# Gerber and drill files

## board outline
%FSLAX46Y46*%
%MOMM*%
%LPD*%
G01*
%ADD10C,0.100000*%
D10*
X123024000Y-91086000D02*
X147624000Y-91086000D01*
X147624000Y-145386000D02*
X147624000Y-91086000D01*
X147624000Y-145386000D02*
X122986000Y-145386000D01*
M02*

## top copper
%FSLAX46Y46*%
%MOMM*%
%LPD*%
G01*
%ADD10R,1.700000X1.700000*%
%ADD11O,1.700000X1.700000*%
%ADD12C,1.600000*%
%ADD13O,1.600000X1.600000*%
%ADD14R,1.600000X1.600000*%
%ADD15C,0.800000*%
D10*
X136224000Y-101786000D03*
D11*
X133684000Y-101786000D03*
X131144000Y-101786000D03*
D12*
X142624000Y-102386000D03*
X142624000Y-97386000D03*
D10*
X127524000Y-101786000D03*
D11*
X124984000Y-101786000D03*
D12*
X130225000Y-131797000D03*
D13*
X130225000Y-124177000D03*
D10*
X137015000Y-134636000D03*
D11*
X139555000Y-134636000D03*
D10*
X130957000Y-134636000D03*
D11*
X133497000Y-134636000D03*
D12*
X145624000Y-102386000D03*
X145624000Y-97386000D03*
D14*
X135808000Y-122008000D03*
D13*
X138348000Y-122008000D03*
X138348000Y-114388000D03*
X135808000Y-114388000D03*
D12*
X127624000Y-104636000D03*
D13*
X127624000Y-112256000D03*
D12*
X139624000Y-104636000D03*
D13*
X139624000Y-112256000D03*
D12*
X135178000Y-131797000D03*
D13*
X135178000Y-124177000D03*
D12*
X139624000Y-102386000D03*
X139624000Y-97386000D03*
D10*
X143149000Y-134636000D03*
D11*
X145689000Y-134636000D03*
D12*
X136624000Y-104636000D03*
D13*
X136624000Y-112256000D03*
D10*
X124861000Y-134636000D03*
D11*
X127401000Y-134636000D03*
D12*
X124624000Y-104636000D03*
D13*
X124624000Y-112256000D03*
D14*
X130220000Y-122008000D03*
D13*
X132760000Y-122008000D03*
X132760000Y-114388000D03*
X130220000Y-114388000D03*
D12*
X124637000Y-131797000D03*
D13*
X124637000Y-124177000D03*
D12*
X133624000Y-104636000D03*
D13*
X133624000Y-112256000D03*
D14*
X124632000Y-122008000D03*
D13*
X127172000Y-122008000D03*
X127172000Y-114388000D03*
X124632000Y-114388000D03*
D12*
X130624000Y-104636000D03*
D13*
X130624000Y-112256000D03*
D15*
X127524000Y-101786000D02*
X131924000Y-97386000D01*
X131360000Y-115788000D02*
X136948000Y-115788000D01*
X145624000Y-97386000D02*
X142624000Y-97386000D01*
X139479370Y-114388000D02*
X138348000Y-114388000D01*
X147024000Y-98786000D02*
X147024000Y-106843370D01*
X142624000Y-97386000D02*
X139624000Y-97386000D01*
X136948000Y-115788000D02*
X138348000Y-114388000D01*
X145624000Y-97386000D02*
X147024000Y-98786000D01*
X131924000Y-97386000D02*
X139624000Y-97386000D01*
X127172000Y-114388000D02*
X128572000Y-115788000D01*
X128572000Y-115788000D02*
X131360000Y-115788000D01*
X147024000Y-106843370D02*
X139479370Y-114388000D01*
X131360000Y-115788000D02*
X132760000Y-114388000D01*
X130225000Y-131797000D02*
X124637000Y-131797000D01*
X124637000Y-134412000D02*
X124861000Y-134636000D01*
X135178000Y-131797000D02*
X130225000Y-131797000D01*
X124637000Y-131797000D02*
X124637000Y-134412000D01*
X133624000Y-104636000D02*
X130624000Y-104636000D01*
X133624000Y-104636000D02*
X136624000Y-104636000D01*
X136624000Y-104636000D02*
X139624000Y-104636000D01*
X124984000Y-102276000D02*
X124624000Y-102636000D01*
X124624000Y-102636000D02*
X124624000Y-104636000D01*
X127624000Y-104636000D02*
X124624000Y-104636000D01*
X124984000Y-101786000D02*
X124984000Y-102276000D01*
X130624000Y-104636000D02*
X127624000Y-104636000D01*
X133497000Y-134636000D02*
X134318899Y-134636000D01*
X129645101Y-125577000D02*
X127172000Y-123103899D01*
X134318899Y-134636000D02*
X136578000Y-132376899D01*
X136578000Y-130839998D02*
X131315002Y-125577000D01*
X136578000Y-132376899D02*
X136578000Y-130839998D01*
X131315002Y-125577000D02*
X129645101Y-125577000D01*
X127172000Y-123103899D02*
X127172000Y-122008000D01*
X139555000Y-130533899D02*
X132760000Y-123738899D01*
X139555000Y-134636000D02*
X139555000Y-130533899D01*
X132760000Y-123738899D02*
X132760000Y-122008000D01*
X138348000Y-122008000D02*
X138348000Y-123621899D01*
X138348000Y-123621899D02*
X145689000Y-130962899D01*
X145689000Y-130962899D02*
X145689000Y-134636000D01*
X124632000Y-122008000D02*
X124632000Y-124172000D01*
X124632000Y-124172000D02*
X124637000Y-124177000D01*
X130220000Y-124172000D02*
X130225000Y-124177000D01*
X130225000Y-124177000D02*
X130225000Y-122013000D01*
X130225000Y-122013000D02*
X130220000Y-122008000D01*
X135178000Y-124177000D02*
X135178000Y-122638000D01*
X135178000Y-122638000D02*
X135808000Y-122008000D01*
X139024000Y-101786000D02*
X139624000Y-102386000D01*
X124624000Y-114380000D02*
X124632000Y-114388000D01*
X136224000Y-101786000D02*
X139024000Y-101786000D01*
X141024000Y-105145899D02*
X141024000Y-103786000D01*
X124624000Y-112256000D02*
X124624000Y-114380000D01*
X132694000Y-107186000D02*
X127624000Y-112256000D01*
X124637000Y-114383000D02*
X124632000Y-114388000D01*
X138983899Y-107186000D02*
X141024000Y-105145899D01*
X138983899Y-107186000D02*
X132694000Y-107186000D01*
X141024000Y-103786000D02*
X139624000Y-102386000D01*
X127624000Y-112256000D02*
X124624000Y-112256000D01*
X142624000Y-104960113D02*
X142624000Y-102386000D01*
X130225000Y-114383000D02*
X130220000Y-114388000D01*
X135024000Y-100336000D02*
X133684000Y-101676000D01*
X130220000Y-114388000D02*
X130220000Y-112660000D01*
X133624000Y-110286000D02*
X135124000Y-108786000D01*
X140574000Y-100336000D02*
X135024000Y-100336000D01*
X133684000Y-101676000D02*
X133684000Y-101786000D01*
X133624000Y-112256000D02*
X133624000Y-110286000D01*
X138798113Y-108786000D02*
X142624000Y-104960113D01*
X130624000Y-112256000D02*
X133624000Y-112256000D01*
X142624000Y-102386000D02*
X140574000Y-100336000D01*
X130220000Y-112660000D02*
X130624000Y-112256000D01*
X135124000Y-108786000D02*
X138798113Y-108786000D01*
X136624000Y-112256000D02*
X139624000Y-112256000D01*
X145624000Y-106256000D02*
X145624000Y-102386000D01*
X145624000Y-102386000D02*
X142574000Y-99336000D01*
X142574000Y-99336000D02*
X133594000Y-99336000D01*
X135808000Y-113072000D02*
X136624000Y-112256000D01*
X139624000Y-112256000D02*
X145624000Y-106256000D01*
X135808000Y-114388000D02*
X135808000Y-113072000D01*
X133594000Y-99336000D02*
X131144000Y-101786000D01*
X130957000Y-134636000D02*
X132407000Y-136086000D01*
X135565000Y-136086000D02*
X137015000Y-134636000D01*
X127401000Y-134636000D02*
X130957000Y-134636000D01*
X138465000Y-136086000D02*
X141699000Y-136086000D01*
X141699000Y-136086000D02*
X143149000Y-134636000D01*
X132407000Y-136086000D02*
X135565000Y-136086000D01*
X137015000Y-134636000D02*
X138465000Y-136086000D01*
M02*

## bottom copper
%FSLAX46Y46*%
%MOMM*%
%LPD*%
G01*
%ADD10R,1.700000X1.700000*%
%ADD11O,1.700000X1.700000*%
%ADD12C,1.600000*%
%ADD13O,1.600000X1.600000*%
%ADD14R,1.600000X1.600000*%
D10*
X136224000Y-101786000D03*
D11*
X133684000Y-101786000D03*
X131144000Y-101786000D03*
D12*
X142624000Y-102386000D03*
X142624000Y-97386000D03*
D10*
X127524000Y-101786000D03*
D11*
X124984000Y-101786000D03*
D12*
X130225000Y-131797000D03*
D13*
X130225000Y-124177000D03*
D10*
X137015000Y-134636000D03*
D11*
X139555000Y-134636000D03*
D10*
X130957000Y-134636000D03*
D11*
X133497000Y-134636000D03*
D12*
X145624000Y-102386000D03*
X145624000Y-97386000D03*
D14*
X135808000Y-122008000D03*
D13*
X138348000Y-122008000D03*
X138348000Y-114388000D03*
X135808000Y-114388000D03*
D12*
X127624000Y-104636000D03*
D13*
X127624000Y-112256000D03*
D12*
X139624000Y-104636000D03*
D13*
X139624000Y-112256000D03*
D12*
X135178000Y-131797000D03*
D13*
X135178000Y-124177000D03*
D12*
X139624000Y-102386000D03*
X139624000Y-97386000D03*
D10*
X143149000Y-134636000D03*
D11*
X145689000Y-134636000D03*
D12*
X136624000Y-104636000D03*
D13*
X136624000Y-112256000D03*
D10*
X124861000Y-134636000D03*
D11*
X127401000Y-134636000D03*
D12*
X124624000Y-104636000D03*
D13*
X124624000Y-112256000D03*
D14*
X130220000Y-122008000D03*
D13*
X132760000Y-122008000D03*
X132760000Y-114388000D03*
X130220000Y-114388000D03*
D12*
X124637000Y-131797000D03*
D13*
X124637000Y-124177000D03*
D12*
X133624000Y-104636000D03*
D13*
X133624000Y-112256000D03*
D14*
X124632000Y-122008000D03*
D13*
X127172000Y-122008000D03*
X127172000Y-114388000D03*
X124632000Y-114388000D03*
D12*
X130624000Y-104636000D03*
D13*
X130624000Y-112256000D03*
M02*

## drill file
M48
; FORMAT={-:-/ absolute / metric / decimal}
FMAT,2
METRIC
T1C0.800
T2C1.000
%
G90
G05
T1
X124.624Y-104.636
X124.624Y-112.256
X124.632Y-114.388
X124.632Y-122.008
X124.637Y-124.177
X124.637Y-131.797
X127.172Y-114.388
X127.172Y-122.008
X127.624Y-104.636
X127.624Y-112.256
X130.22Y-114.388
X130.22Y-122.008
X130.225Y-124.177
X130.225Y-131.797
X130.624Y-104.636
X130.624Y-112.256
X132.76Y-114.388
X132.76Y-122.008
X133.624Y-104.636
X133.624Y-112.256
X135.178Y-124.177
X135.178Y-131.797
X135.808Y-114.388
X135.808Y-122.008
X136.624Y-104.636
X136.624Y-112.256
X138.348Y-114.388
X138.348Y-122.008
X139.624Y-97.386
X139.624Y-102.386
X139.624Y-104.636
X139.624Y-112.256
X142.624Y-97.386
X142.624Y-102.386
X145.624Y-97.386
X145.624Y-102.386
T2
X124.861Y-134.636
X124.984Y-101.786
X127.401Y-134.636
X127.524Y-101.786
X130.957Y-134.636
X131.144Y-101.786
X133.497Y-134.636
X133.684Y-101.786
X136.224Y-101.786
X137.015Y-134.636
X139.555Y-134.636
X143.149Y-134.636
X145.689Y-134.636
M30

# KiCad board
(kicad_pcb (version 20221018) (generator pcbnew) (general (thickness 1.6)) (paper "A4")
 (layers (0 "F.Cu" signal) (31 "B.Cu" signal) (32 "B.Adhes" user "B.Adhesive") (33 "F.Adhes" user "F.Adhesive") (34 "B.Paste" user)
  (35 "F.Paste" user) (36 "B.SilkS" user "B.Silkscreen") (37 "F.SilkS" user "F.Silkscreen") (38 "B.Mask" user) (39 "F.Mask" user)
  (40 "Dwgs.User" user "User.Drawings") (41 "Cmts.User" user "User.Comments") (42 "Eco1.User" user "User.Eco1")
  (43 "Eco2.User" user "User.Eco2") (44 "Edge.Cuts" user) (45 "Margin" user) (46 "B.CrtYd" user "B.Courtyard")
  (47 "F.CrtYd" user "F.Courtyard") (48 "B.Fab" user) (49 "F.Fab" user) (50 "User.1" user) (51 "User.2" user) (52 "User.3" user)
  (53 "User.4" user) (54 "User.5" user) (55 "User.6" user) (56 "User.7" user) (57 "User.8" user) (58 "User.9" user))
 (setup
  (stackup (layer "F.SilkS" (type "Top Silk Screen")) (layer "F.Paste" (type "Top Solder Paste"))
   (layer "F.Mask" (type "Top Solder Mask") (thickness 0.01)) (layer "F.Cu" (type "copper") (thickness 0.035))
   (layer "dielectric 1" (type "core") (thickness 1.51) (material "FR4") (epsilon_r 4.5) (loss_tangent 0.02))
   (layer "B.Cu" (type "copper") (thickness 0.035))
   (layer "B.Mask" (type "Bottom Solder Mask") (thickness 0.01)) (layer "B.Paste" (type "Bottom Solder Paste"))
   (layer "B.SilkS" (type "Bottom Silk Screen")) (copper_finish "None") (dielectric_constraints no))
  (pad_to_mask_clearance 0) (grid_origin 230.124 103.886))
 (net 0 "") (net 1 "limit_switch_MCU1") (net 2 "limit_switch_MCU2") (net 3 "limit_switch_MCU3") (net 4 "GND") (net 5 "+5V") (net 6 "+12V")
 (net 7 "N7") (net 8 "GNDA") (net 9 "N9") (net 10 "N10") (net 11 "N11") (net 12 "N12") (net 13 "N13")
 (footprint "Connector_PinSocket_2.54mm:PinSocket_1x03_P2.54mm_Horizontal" (layer "F.Cu") (at 136.224 101.786 -90)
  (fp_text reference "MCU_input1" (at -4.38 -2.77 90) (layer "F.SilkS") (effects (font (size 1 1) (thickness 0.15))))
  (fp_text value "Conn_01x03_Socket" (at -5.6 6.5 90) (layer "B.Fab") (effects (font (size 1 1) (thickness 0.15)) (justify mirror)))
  (pad "1" thru_hole rect (at 0 0 270) (size 1.7 1.7) (drill 1) (layers "*.Cu" "*.Mask") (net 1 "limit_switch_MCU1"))
  (pad "2" thru_hole oval (at 0 2.54 270) (size 1.7 1.7) (drill 1) (layers "*.Cu" "*.Mask") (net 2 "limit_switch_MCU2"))
  (pad "3" thru_hole oval (at 0 5.08 270) (size 1.7 1.7) (drill 1) (layers "*.Cu" "*.Mask") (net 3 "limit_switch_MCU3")))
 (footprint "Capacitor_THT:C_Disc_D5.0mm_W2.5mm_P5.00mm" (layer "F.Cu") (at 142.624 102.386 90)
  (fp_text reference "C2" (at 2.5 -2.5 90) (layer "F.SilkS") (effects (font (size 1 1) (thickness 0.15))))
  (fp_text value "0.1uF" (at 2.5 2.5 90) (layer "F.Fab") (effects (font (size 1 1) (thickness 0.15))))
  (pad "1" thru_hole circle (at 0 0 90) (size 1.6 1.6) (drill 0.8) (layers "*.Cu" "*.Mask") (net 2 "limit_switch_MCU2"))
  (pad "2" thru_hole circle (at 5 0 90) (size 1.6 1.6) (drill 0.8) (layers "*.Cu" "*.Mask") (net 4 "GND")))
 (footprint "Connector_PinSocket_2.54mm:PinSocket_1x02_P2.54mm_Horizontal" (layer "F.Cu") (at 127.524 101.786 -90)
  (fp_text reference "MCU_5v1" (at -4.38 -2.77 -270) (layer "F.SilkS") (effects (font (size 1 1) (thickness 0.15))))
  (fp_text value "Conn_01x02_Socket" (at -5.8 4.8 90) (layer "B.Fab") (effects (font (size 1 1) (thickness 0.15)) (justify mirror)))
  (pad "1" thru_hole rect (at 0 0 270) (size 1.7 1.7) (drill 1) (layers "*.Cu" "*.Mask") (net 4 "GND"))
  (pad "2" thru_hole oval (at 0 2.54 270) (size 1.7 1.7) (drill 1) (layers "*.Cu" "*.Mask") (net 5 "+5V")))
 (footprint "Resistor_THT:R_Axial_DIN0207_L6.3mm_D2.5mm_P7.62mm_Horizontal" (layer "F.Cu") (at 130.225 131.797 90)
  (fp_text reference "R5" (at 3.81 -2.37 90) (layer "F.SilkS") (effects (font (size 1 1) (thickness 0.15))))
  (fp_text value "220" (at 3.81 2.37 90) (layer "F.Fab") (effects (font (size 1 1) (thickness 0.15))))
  (pad "1" thru_hole circle (at 0 0 90) (size 1.6 1.6) (drill 0.8) (layers "*.Cu" "*.Mask") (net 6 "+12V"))
  (pad "2" thru_hole oval (at 7.62 0 90) (size 1.6 1.6) (drill 0.8) (layers "*.Cu" "*.Mask") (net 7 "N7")))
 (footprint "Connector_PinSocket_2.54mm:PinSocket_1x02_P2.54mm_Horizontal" (layer "F.Cu") (at 137.015 134.636 90)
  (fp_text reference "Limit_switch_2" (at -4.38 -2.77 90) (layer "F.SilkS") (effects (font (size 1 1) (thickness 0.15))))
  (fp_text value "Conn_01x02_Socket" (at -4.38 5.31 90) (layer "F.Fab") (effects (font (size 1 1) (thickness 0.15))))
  (pad "1" thru_hole rect (at 0 0 90) (size 1.7 1.7) (drill 1) (layers "*.Cu" "*.Mask") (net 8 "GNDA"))
  (pad "2" thru_hole oval (at 0 2.54 90) (size 1.7 1.7) (drill 1) (layers "*.Cu" "*.Mask") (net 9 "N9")))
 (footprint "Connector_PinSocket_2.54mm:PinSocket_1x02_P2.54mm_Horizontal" (layer "F.Cu") (at 130.957 134.636 90)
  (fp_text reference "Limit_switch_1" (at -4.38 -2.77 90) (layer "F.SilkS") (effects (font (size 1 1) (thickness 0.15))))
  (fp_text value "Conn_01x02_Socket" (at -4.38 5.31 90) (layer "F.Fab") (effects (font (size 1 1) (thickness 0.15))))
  (pad "1" thru_hole rect (at 0 0 90) (size 1.7 1.7) (drill 1) (layers "*.Cu" "*.Mask") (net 8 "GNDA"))
  (pad "2" thru_hole oval (at 0 2.54 90) (size 1.7 1.7) (drill 1) (layers "*.Cu" "*.Mask") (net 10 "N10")))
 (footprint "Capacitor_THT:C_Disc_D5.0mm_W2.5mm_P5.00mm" (layer "F.Cu") (at 145.624 102.386 90)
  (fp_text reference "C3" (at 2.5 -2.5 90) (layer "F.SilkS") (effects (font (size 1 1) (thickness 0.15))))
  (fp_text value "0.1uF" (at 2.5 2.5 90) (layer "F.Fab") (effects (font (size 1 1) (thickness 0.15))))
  (pad "1" thru_hole circle (at 0 0 90) (size 1.6 1.6) (drill 0.8) (layers "*.Cu" "*.Mask") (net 3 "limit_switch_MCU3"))
  (pad "2" thru_hole circle (at 5 0 90) (size 1.6 1.6) (drill 0.8) (layers "*.Cu" "*.Mask") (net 4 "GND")))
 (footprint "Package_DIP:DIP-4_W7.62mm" (layer "F.Cu") (at 135.808 122.008 90)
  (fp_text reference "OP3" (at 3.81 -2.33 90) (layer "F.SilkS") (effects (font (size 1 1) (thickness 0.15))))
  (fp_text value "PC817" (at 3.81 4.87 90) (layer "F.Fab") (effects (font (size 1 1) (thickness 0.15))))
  (pad "1" thru_hole rect (at 0 0 90) (size 1.6 1.6) (drill 0.8) (layers "*.Cu" "*.Mask") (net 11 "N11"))
  (pad "2" thru_hole oval (at 0 2.54 90) (size 1.6 1.6) (drill 0.8) (layers "*.Cu" "*.Mask") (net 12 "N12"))
  (pad "3" thru_hole oval (at 7.62 2.54 90) (size 1.6 1.6) (drill 0.8) (layers "*.Cu" "*.Mask") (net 4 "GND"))
  (pad "4" thru_hole oval (at 7.62 0 90) (size 1.6 1.6) (drill 0.8) (layers "*.Cu" "*.Mask") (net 3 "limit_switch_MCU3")))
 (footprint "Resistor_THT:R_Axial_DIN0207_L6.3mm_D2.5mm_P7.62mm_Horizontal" (layer "F.Cu") (at 127.624 104.636 -90)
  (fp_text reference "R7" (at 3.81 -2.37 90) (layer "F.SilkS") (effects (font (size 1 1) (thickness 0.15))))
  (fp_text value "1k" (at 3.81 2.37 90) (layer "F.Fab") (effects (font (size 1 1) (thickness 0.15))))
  (pad "1" thru_hole circle (at 0 0 270) (size 1.6 1.6) (drill 0.8) (layers "*.Cu" "*.Mask") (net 5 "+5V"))
  (pad "2" thru_hole oval (at 7.62 0 270) (size 1.6 1.6) (drill 0.8) (layers "*.Cu" "*.Mask") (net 1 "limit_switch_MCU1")))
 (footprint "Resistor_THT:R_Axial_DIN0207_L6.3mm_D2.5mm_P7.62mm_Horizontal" (layer "F.Cu") (at 139.624 104.636 -90)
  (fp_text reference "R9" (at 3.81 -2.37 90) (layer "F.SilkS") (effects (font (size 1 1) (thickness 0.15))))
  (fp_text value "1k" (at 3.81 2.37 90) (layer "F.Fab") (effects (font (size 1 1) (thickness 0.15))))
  (pad "1" thru_hole circle (at 0 0 270) (size 1.6 1.6) (drill 0.8) (layers "*.Cu" "*.Mask") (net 5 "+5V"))
  (pad "2" thru_hole oval (at 7.62 0 270) (size 1.6 1.6) (drill 0.8) (layers "*.Cu" "*.Mask") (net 3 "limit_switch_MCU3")))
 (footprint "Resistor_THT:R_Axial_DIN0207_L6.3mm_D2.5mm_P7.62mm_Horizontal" (layer "F.Cu") (at 135.178 131.797 90)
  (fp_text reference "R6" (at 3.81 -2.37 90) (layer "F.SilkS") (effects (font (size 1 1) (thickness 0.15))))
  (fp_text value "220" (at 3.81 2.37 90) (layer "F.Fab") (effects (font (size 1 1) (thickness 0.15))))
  (pad "1" thru_hole circle (at 0 0 90) (size 1.6 1.6) (drill 0.8) (layers "*.Cu" "*.Mask") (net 6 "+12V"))
  (pad "2" thru_hole oval (at 7.62 0 90) (size 1.6 1.6) (drill 0.8) (layers "*.Cu" "*.Mask") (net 11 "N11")))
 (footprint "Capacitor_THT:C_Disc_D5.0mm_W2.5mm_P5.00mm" (layer "F.Cu") (at 139.624 102.386 90)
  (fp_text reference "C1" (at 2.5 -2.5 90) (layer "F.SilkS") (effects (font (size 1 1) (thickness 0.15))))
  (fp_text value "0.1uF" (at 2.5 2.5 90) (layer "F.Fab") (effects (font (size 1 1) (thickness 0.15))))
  (pad "1" thru_hole circle (at 0 0 90) (size 1.6 1.6) (drill 0.8) (layers "*.Cu" "*.Mask") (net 1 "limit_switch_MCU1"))
  (pad "2" thru_hole circle (at 5 0 90) (size 1.6 1.6) (drill 0.8) (layers "*.Cu" "*.Mask") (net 4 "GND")))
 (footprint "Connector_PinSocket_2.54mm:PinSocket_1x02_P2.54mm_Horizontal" (layer "F.Cu") (at 143.149 134.636 90)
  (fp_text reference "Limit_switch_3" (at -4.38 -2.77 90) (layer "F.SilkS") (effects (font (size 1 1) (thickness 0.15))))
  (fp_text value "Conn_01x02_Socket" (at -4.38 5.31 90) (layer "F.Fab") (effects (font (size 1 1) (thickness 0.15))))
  (pad "1" thru_hole rect (at 0 0 90) (size 1.7 1.7) (drill 1) (layers "*.Cu" "*.Mask") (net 8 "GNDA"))
  (pad "2" thru_hole oval (at 0 2.54 90) (size 1.7 1.7) (drill 1) (layers "*.Cu" "*.Mask") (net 12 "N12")))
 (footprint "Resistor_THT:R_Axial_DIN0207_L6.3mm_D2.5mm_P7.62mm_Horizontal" (layer "F.Cu") (at 136.624 104.636 -90)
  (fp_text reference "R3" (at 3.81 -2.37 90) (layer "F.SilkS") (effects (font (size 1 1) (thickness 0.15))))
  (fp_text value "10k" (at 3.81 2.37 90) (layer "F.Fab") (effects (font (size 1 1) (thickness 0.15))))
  (pad "1" thru_hole circle (at 0 0 270) (size 1.6 1.6) (drill 0.8) (layers "*.Cu" "*.Mask") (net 5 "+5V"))
  (pad "2" thru_hole oval (at 7.62 0 270) (size 1.6 1.6) (drill 0.8) (layers "*.Cu" "*.Mask") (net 3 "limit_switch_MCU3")))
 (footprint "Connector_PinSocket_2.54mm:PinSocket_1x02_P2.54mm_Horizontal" (layer "F.Cu") (at 124.861 134.636 90)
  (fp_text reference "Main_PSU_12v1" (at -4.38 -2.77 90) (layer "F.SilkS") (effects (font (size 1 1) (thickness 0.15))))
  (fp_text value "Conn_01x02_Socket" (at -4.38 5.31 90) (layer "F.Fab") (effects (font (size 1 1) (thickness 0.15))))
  (pad "1" thru_hole rect (at 0 0 90) (size 1.7 1.7) (drill 1) (layers "*.Cu" "*.Mask") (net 6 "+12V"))
  (pad "2" thru_hole oval (at 0 2.54 90) (size 1.7 1.7) (drill 1) (layers "*.Cu" "*.Mask") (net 8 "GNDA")))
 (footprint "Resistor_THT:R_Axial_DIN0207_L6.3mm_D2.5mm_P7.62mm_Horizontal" (layer "F.Cu") (at 124.624 104.636 -90)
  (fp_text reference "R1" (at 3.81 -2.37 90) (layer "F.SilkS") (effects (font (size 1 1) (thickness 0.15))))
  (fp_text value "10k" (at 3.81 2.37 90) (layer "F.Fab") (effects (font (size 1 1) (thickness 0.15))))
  (pad "1" thru_hole circle (at 0 0 270) (size 1.6 1.6) (drill 0.8) (layers "*.Cu" "*.Mask") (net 5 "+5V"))
  (pad "2" thru_hole oval (at 7.62 0 270) (size 1.6 1.6) (drill 0.8) (layers "*.Cu" "*.Mask") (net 1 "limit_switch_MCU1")))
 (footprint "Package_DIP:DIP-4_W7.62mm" (layer "F.Cu") (at 130.22 122.008 90)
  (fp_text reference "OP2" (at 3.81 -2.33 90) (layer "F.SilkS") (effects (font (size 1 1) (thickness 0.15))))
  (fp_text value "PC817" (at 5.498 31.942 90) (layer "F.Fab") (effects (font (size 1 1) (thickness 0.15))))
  (pad "1" thru_hole rect (at 0 0 90) (size 1.6 1.6) (drill 0.8) (layers "*.Cu" "*.Mask") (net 7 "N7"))
  (pad "2" thru_hole oval (at 0 2.54 90) (size 1.6 1.6) (drill 0.8) (layers "*.Cu" "*.Mask") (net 9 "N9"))
  (pad "3" thru_hole oval (at 7.62 2.54 90) (size 1.6 1.6) (drill 0.8) (layers "*.Cu" "*.Mask") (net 4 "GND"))
  (pad "4" thru_hole oval (at 7.62 0 90) (size 1.6 1.6) (drill 0.8) (layers "*.Cu" "*.Mask") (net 2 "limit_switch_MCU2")))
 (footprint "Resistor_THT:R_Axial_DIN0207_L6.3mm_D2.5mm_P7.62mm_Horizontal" (layer "F.Cu") (at 124.637 131.797 90)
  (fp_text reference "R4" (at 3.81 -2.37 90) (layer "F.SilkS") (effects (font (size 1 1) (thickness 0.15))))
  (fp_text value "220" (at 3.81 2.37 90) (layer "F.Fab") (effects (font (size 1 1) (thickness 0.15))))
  (pad "1" thru_hole circle (at 0 0 90) (size 1.6 1.6) (drill 0.8) (layers "*.Cu" "*.Mask") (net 6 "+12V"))
  (pad "2" thru_hole oval (at 7.62 0 90) (size 1.6 1.6) (drill 0.8) (layers "*.Cu" "*.Mask") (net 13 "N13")))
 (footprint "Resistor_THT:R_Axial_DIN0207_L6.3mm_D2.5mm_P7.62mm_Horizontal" (layer "F.Cu") (at 133.624 104.636 -90)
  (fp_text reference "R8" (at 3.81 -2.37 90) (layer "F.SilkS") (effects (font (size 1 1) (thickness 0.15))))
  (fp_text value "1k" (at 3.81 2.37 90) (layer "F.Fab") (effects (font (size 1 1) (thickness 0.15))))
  (pad "1" thru_hole circle (at 0 0 270) (size 1.6 1.6) (drill 0.8) (layers "*.Cu" "*.Mask") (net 5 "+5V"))
  (pad "2" thru_hole oval (at 7.62 0 270) (size 1.6 1.6) (drill 0.8) (layers "*.Cu" "*.Mask") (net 2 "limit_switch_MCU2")))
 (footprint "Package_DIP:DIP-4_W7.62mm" (layer "F.Cu") (at 124.632 122.008 90)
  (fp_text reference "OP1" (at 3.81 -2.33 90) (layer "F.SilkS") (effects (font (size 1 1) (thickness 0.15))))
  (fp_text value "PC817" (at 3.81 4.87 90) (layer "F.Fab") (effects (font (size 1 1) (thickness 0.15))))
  (pad "1" thru_hole rect (at 0 0 90) (size 1.6 1.6) (drill 0.8) (layers "*.Cu" "*.Mask") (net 13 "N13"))
  (pad "2" thru_hole oval (at 0 2.54 90) (size 1.6 1.6) (drill 0.8) (layers "*.Cu" "*.Mask") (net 10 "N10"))
  (pad "3" thru_hole oval (at 7.62 2.54 90) (size 1.6 1.6) (drill 0.8) (layers "*.Cu" "*.Mask") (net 4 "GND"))
  (pad "4" thru_hole oval (at 7.62 0 90) (size 1.6 1.6) (drill 0.8) (layers "*.Cu" "*.Mask") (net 1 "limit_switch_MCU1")))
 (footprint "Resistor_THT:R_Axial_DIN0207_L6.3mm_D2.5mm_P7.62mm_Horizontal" (layer "F.Cu") (at 130.624 104.636 -90)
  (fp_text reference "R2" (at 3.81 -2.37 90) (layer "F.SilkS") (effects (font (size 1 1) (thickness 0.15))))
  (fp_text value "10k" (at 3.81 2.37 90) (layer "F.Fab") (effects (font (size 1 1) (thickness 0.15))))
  (pad "1" thru_hole circle (at 0 0 270) (size 1.6 1.6) (drill 0.8) (layers "*.Cu" "*.Mask") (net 5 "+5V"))
  (pad "2" thru_hole oval (at 7.62 0 270) (size 1.6 1.6) (drill 0.8) (layers "*.Cu" "*.Mask") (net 2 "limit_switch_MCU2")))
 (gr_line (start 123.024 91.086) (end 147.624 91.086) (stroke (width 0.1) (type default)) (layer "Edge.Cuts"))
 (gr_line (start 147.624 145.386) (end 147.624 91.086) (stroke (width 0.1) (type default)) (layer "Edge.Cuts"))
 (gr_line (start 147.624 145.386) (end 122.986 145.386) (stroke (width 0.1) (type default)) (layer "Edge.Cuts"))
 (segment (start 127.524 101.786) (end 131.924 97.386) (width 0.8) (layer "F.Cu") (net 4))
 (segment (start 131.36 115.788) (end 136.948 115.788) (width 0.8) (layer "F.Cu") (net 4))
 (segment (start 145.624 97.386) (end 142.624 97.386) (width 0.8) (layer "F.Cu") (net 4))
 (segment (start 139.47937 114.388) (end 138.348 114.388) (width 0.8) (layer "F.Cu") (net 4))
 (segment (start 147.024 98.786) (end 147.024 106.84337) (width 0.8) (layer "F.Cu") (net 4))
 (segment (start 142.624 97.386) (end 139.624 97.386) (width 0.8) (layer "F.Cu") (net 4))
 (segment (start 136.948 115.788) (end 138.348 114.388) (width 0.8) (layer "F.Cu") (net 4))
 (segment (start 145.624 97.386) (end 147.024 98.786) (width 0.8) (layer "F.Cu") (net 4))
 (segment (start 131.924 97.386) (end 139.624 97.386) (width 0.8) (layer "F.Cu") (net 4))
 (segment (start 127.172 114.388) (end 128.572 115.788) (width 0.8) (layer "F.Cu") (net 4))
 (segment (start 128.572 115.788) (end 131.36 115.788) (width 0.8) (layer "F.Cu") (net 4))
 (segment (start 147.024 106.84337) (end 139.47937 114.388) (width 0.8) (layer "F.Cu") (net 4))
 (segment (start 131.36 115.788) (end 132.76 114.388) (width 0.8) (layer "F.Cu") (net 4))
 (segment (start 130.225 131.797) (end 124.637 131.797) (width 0.8) (layer "F.Cu") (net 6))
 (segment (start 124.637 134.412) (end 124.861 134.636) (width 0.8) (layer "F.Cu") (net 6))
 (segment (start 135.178 131.797) (end 130.225 131.797) (width 0.8) (layer "F.Cu") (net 6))
 (segment (start 124.637 131.797) (end 124.637 134.412) (width 0.8) (layer "F.Cu") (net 6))
 (segment (start 133.624 104.636) (end 130.624 104.636) (width 0.8) (layer "F.Cu") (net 5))
 (segment (start 133.624 104.636) (end 136.624 104.636) (width 0.8) (layer "F.Cu") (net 5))
 (segment (start 136.624 104.636) (end 139.624 104.636) (width 0.8) (layer "F.Cu") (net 5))
 (segment (start 124.984 102.276) (end 124.624 102.636) (width 0.8) (layer "F.Cu") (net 5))
 (segment (start 124.624 102.636) (end 124.624 104.636) (width 0.8) (layer "F.Cu") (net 5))
 (segment (start 127.624 104.636) (end 124.624 104.636) (width 0.8) (layer "F.Cu") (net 5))
 (segment (start 124.984 101.786) (end 124.984 102.276) (width 0.8) (layer "F.Cu") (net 5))
 (segment (start 130.624 104.636) (end 127.624 104.636) (width 0.8) (layer "F.Cu") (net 5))
 (segment (start 133.497 134.636) (end 134.318899 134.636) (width 0.8) (layer "F.Cu") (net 10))
 (segment (start 129.645101 125.577) (end 127.172 123.103899) (width 0.8) (layer "F.Cu") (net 10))
 (segment (start 134.318899 134.636) (end 136.578 132.376899) (width 0.8) (layer "F.Cu") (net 10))
 (segment (start 136.578 130.839998) (end 131.315002 125.577) (width 0.8) (layer "F.Cu") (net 10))
 (segment (start 136.578 132.376899) (end 136.578 130.839998) (width 0.8) (layer "F.Cu") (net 10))
 (segment (start 131.315002 125.577) (end 129.645101 125.577) (width 0.8) (layer "F.Cu") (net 10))
 (segment (start 127.172 123.103899) (end 127.172 122.008) (width 0.8) (layer "F.Cu") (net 10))
 (segment (start 139.555 130.533899) (end 132.76 123.738899) (width 0.8) (layer "F.Cu") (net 9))
 (segment (start 139.555 134.636) (end 139.555 130.533899) (width 0.8) (layer "F.Cu") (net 9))
 (segment (start 132.76 123.738899) (end 132.76 122.008) (width 0.8) (layer "F.Cu") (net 9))
 (segment (start 138.348 122.008) (end 138.348 123.621899) (width 0.8) (layer "F.Cu") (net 12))
 (segment (start 138.348 123.621899) (end 145.689 130.962899) (width 0.8) (layer "F.Cu") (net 12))
 (segment (start 145.689 130.962899) (end 145.689 134.636) (width 0.8) (layer "F.Cu") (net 12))
 (segment (start 124.632 122.008) (end 124.632 124.172) (width 0.8) (layer "F.Cu") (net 13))
 (segment (start 124.632 124.172) (end 124.637 124.177) (width 0.8) (layer "F.Cu") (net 13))
 (segment (start 130.22 124.172) (end 130.225 124.177) (width 0.8) (layer "F.Cu") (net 7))
 (segment (start 130.225 124.177) (end 130.225 122.013) (width 0.8) (layer "F.Cu") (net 7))
 (segment (start 130.225 122.013) (end 130.22 122.008) (width 0.8) (layer "F.Cu") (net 7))
 (segment (start 135.178 124.177) (end 135.178 122.638) (width 0.8) (layer "F.Cu") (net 11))
 (segment (start 135.178 122.638) (end 135.808 122.008) (width 0.8) (layer "F.Cu") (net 11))
 (segment (start 139.024 101.786) (end 139.624 102.386) (width 0.8) (layer "F.Cu") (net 1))
 (segment (start 124.624 114.38) (end 124.632 114.388) (width 0.8) (layer "F.Cu") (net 1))
 (segment (start 136.224 101.786) (end 139.024 101.786) (width 0.8) (layer "F.Cu") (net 1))
 (segment (start 141.024 105.145899) (end 141.024 103.786) (width 0.8) (layer "F.Cu") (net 1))
 (segment (start 124.624 112.256) (end 124.624 114.38) (width 0.8) (layer "F.Cu") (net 1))
 (segment (start 132.694 107.186) (end 127.624 112.256) (width 0.8) (layer "F.Cu") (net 1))
 (segment (start 124.637 114.383) (end 124.632 114.388) (width 0.8) (layer "F.Cu") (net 1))
 (segment (start 138.983899 107.186) (end 141.024 105.145899) (width 0.8) (layer "F.Cu") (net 1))
 (segment (start 138.983899 107.186) (end 132.694 107.186) (width 0.8) (layer "F.Cu") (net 1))
 (segment (start 141.024 103.786) (end 139.624 102.386) (width 0.8) (layer "F.Cu") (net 1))
 (segment (start 127.624 112.256) (end 124.624 112.256) (width 0.8) (layer "F.Cu") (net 1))
 (segment (start 142.624 104.960113) (end 142.624 102.386) (width 0.8) (layer "F.Cu") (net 2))
 (segment (start 130.225 114.383) (end 130.22 114.388) (width 0.8) (layer "F.Cu") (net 2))
 (segment (start 135.024 100.336) (end 133.684 101.676) (width 0.8) (layer "F.Cu") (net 2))
 (segment (start 130.22 114.388) (end 130.22 112.66) (width 0.8) (layer "F.Cu") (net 2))
 (segment (start 133.624 110.286) (end 135.124 108.786) (width 0.8) (layer "F.Cu") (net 2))
 (segment (start 140.574 100.336) (end 135.024 100.336) (width 0.8) (layer "F.Cu") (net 2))
 (segment (start 133.684 101.676) (end 133.684 101.786) (width 0.8) (layer "F.Cu") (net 2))
 (segment (start 133.624 112.256) (end 133.624 110.286) (width 0.8) (layer "F.Cu") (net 2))
 (segment (start 138.798113 108.786) (end 142.624 104.960113) (width 0.8) (layer "F.Cu") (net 2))
 (segment (start 130.624 112.256) (end 133.624 112.256) (width 0.8) (layer "F.Cu") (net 2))
 (segment (start 142.624 102.386) (end 140.574 100.336) (width 0.8) (layer "F.Cu") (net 2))
 (segment (start 130.22 112.66) (end 130.624 112.256) (width 0.8) (layer "F.Cu") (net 2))
 (segment (start 135.124 108.786) (end 138.798113 108.786) (width 0.8) (layer "F.Cu") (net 2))
 (segment (start 136.624 112.256) (end 139.624 112.256) (width 0.8) (layer "F.Cu") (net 3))
 (segment (start 145.624 106.256) (end 145.624 102.386) (width 0.8) (layer "F.Cu") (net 3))
 (segment (start 145.624 102.386) (end 142.574 99.336) (width 0.8) (layer "F.Cu") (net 3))
 (segment (start 142.574 99.336) (end 133.594 99.336) (width 0.8) (layer "F.Cu") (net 3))
 (segment (start 135.808 113.072) (end 136.624 112.256) (width 0.8) (layer "F.Cu") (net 3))
 (segment (start 139.624 112.256) (end 145.624 106.256) (width 0.8) (layer "F.Cu") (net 3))
 (segment (start 135.808 114.388) (end 135.808 113.072) (width 0.8) (layer "F.Cu") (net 3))
 (segment (start 133.594 99.336) (end 131.144 101.786) (width 0.8) (layer "F.Cu") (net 3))
 (segment (start 130.957 134.636) (end 132.407 136.086) (width 0.8) (layer "F.Cu") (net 8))
 (segment (start 135.565 136.086) (end 137.015 134.636) (width 0.8) (layer "F.Cu") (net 8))
 (segment (start 127.401 134.636) (end 130.957 134.636) (width 0.8) (layer "F.Cu") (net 8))
 (segment (start 138.465 136.086) (end 141.699 136.086) (width 0.8) (layer "F.Cu") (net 8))
 (segment (start 141.699 136.086) (end 143.149 134.636) (width 0.8) (layer "F.Cu") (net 8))
 (segment (start 132.407 136.086) (end 135.565 136.086) (width 0.8) (layer "F.Cu") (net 8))
 (segment (start 137.015 134.636) (end 138.465 136.086) (width 0.8) (layer "F.Cu") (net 8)))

